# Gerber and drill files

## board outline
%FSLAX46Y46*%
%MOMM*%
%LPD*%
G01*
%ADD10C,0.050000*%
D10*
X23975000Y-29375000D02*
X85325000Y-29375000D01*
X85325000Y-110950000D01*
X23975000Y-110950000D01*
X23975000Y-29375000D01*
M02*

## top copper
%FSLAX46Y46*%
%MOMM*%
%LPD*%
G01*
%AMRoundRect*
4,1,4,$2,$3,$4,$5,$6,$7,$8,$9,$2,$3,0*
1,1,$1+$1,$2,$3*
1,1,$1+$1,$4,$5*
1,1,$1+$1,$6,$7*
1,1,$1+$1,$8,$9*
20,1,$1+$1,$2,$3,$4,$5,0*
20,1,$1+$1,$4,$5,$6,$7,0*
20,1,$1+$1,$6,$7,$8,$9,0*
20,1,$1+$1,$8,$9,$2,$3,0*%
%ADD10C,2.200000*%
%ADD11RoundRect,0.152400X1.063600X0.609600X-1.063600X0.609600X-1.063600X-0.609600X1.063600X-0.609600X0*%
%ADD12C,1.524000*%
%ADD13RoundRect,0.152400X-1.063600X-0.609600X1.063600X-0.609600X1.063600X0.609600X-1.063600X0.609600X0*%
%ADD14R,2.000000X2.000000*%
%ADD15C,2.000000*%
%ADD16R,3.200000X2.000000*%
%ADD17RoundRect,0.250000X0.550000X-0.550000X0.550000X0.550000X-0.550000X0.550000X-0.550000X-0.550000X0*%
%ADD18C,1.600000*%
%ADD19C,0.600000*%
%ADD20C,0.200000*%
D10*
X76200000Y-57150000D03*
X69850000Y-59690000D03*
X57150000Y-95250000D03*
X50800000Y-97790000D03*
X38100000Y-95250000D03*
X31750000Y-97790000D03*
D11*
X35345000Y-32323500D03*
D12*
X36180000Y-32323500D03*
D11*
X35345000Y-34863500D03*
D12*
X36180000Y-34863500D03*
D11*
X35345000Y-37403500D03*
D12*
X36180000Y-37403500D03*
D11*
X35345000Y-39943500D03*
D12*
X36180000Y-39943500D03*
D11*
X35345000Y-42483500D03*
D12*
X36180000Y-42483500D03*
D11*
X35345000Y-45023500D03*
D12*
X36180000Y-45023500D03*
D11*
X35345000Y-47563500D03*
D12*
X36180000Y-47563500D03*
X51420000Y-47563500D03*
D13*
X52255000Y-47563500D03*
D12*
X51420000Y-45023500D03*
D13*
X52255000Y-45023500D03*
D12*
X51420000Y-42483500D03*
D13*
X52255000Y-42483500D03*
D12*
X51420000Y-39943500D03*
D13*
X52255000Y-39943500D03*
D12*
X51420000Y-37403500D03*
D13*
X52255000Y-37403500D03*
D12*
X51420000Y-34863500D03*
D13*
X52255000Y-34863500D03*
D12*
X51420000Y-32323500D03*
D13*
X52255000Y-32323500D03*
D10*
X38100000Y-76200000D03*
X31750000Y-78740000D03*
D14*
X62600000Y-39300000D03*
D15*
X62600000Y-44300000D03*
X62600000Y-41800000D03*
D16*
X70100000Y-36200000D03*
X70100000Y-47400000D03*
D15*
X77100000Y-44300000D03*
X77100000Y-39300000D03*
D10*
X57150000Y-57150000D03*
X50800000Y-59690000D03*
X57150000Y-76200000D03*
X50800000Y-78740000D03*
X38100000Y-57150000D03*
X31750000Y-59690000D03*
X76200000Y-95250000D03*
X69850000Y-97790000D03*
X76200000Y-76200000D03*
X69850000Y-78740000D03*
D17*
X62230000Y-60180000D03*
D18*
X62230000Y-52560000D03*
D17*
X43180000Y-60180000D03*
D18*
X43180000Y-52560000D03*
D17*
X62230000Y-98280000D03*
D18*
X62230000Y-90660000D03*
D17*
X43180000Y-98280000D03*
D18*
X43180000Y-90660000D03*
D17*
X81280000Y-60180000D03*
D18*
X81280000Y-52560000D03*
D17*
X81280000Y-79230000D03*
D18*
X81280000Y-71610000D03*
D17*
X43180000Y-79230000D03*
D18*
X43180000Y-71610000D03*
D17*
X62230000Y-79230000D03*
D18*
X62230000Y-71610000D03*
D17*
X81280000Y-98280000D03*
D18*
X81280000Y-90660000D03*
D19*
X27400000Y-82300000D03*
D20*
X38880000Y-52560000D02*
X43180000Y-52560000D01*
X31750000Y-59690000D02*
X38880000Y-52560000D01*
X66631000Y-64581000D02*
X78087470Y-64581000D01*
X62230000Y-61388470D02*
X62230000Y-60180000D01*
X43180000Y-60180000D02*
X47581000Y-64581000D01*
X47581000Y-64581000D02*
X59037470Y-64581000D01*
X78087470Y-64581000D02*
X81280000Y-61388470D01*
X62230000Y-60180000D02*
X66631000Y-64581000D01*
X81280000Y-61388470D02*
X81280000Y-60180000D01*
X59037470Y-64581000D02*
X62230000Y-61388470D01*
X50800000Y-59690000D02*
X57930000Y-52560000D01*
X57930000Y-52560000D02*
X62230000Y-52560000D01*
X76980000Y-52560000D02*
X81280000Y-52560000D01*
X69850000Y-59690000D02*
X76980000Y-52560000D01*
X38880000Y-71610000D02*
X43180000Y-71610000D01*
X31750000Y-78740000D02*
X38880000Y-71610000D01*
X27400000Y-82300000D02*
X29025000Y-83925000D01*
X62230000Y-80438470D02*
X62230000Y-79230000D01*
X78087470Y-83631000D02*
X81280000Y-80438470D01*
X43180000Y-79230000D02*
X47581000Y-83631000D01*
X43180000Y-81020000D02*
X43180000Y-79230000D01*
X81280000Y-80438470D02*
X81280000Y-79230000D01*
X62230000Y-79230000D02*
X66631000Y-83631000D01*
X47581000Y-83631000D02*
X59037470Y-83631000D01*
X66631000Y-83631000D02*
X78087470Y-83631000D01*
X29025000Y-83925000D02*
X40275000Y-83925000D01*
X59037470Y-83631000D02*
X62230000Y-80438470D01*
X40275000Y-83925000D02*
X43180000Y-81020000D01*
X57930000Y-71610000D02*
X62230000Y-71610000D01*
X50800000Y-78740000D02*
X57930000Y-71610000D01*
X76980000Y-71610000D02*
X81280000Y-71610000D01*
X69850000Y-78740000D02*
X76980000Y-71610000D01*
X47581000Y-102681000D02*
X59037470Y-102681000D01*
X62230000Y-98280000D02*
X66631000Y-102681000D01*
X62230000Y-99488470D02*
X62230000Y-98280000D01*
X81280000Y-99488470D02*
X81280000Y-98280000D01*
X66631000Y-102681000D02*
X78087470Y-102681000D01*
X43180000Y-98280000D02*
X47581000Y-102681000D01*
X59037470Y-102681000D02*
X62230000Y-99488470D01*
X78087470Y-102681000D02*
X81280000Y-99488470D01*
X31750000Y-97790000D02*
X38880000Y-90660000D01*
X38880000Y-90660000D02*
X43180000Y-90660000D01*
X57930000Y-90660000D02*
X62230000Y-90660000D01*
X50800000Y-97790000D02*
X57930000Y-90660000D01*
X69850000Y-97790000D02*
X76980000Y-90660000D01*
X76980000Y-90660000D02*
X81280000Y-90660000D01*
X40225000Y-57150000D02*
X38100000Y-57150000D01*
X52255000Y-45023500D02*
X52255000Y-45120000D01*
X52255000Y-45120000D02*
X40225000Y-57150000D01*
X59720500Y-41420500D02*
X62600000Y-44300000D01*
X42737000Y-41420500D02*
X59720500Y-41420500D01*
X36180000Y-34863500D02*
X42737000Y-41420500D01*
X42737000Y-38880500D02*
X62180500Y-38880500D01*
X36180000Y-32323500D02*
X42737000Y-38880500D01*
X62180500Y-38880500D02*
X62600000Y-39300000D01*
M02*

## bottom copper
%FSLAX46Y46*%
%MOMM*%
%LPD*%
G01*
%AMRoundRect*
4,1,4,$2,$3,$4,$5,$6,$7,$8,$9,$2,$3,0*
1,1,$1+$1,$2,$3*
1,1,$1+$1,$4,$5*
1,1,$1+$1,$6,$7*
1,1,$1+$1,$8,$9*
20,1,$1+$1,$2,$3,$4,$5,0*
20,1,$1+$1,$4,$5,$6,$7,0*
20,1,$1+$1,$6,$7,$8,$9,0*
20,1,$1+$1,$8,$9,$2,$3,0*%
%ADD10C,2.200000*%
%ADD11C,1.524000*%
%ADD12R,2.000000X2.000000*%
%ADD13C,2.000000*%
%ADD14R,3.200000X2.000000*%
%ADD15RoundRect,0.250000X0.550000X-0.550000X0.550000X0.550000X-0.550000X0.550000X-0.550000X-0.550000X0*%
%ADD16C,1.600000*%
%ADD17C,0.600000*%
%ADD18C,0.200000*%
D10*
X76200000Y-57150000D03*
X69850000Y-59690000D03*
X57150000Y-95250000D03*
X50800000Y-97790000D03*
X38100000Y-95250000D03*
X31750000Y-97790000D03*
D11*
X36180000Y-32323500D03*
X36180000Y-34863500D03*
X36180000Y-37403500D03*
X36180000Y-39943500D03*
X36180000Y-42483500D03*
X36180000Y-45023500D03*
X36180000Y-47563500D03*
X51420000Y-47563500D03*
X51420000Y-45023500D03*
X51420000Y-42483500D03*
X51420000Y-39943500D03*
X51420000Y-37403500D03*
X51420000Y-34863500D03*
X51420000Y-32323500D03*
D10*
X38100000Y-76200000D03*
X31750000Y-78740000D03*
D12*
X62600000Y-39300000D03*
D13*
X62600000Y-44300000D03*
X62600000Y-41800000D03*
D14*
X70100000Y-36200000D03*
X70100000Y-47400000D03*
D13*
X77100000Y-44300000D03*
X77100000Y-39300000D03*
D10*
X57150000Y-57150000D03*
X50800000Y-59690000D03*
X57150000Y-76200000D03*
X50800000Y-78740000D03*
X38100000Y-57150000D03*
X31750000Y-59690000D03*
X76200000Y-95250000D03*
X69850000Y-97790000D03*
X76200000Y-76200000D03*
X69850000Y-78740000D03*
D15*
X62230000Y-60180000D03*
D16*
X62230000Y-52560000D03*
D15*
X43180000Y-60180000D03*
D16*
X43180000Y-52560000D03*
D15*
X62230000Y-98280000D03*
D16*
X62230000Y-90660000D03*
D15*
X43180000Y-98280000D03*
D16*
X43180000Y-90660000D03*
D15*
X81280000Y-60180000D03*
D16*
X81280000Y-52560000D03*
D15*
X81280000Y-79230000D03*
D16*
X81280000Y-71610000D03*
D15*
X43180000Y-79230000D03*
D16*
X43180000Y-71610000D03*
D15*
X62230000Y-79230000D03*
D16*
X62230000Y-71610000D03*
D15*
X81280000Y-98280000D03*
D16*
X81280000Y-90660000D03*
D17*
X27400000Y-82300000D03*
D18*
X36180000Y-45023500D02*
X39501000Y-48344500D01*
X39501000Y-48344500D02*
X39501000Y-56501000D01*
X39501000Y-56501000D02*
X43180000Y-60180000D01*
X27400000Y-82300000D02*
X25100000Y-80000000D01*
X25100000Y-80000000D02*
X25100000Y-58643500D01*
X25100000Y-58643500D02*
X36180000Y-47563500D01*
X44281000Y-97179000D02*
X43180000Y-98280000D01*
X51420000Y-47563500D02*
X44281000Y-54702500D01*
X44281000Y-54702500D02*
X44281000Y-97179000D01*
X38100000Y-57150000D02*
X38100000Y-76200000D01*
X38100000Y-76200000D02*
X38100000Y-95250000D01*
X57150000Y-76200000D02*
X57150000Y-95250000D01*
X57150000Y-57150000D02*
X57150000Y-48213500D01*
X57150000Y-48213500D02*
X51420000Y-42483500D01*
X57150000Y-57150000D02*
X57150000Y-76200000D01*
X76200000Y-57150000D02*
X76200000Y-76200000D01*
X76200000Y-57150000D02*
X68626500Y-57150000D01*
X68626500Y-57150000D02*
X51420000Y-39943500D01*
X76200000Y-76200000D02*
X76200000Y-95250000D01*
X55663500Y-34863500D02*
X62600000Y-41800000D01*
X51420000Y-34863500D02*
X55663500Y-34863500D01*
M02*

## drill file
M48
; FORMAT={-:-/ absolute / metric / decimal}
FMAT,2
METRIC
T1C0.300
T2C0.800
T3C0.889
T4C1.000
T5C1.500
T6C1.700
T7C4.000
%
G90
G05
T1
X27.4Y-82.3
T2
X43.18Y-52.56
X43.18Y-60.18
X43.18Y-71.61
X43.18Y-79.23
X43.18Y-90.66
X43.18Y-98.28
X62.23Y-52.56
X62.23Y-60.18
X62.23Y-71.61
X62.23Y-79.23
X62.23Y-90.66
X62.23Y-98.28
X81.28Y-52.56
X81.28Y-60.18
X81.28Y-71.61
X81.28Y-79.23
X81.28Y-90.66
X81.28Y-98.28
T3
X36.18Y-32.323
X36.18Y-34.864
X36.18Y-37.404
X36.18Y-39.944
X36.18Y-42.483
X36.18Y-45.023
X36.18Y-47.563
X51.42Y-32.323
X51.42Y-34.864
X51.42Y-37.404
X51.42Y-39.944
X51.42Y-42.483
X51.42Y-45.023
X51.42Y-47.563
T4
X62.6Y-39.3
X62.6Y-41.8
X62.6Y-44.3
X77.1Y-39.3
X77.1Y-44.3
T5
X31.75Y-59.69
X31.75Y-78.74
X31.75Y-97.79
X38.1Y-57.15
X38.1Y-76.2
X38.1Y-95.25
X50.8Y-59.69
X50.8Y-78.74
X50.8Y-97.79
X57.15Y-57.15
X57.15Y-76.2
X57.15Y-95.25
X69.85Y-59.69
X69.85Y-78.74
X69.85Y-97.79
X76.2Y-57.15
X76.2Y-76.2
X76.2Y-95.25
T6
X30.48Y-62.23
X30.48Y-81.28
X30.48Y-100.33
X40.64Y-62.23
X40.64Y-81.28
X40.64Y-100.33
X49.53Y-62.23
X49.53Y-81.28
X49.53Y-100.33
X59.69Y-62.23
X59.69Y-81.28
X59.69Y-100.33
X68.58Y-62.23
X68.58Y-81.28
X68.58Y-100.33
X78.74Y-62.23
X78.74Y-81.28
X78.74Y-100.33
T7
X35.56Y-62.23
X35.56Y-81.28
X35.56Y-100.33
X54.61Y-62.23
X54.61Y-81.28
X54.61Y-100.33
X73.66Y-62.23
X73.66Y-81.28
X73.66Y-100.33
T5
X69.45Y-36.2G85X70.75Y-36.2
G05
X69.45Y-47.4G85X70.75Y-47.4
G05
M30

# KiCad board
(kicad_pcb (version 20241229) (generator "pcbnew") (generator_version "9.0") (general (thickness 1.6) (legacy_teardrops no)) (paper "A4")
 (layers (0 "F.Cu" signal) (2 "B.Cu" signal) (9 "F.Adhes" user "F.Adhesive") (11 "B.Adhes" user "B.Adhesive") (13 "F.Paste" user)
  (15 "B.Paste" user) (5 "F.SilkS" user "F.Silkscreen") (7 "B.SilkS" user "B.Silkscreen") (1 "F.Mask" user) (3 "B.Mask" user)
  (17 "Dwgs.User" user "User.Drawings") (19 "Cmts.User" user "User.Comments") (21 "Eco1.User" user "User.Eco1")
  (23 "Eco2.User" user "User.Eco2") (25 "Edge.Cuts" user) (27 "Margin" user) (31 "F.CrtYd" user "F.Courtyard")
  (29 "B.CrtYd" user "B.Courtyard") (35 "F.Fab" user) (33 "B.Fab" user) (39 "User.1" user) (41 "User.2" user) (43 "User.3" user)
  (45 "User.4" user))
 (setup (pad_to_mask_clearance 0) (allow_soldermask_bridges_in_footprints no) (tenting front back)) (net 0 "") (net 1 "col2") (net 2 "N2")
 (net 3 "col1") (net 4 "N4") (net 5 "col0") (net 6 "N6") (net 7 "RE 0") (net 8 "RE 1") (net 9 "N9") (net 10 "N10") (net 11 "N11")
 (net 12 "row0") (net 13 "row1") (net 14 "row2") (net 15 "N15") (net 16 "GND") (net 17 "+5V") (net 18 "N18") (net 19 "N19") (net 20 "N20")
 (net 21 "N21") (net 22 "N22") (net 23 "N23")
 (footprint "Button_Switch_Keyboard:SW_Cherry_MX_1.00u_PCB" (layer "F.Cu") (at 76.2 57.15)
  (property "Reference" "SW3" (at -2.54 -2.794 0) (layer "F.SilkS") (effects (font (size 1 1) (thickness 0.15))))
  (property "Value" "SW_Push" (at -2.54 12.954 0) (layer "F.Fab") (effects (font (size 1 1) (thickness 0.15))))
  (pad "" np_thru_hole circle (at -7.62 5.08) (size 1.7 1.7) (drill 1.7) (layers "*.Cu" "*.Mask"))
  (pad "" np_thru_hole circle (at -2.54 5.08) (size 4 4) (drill 4) (layers "*.Cu" "*.Mask"))
  (pad "" np_thru_hole circle (at 2.54 5.08) (size 1.7 1.7) (drill 1.7) (layers "*.Cu" "*.Mask"))
  (pad "1" thru_hole circle (at 0 0) (size 2.2 2.2) (drill 1.5) (layers "*.Cu" "*.Mask") (remove_unused_layers no) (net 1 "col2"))
  (pad "2" thru_hole circle (at -6.35 2.54) (size 2.2 2.2) (drill 1.5) (layers "*.Cu" "*.Mask") (remove_unused_layers no) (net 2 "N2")))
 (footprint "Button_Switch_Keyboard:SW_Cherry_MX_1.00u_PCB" (layer "F.Cu") (at 57.15 95.25)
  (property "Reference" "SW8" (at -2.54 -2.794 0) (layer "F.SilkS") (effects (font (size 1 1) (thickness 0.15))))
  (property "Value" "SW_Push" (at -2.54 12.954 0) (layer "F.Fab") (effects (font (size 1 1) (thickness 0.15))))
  (pad "" np_thru_hole circle (at -7.62 5.08) (size 1.7 1.7) (drill 1.7) (layers "*.Cu" "*.Mask"))
  (pad "" np_thru_hole circle (at -2.54 5.08) (size 4 4) (drill 4) (layers "*.Cu" "*.Mask"))
  (pad "" np_thru_hole circle (at 2.54 5.08) (size 1.7 1.7) (drill 1.7) (layers "*.Cu" "*.Mask"))
  (pad "1" thru_hole circle (at 0 0) (size 2.2 2.2) (drill 1.5) (layers "*.Cu" "*.Mask") (remove_unused_layers no) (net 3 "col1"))
  (pad "2" thru_hole circle (at -6.35 2.54) (size 2.2 2.2) (drill 1.5) (layers "*.Cu" "*.Mask") (remove_unused_layers no) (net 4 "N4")))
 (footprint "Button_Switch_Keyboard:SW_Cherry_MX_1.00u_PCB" (layer "F.Cu") (at 38.1 95.25)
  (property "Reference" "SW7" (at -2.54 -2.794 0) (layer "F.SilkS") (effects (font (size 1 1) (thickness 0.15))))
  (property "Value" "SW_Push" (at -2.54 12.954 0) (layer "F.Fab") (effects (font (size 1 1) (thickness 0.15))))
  (pad "" np_thru_hole circle (at -7.62 5.08) (size 1.7 1.7) (drill 1.7) (layers "*.Cu" "*.Mask"))
  (pad "" np_thru_hole circle (at -2.54 5.08) (size 4 4) (drill 4) (layers "*.Cu" "*.Mask"))
  (pad "" np_thru_hole circle (at 2.54 5.08) (size 1.7 1.7) (drill 1.7) (layers "*.Cu" "*.Mask"))
  (pad "1" thru_hole circle (at 0 0) (size 2.2 2.2) (drill 1.5) (layers "*.Cu" "*.Mask") (remove_unused_layers no) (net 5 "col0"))
  (pad "2" thru_hole circle (at -6.35 2.54) (size 2.2 2.2) (drill 1.5) (layers "*.Cu" "*.Mask") (remove_unused_layers no) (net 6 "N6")))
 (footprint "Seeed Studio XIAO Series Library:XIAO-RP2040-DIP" (layer "F.Cu") (at 43.8 39.9435)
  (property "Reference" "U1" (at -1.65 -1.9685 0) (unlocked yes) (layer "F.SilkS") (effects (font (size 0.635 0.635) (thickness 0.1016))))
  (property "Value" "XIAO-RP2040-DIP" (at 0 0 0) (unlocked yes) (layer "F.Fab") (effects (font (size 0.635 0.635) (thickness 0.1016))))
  (pad "1" smd roundrect (at -8.455 -7.62 180) (size 2.432 1.524) (layers "F.Cu" "F.Mask") (roundrect_rratio 0.1) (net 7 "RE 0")
   (thermal_bridge_angle 45))
  (pad "1" thru_hole circle (at -7.62 -7.62 180) (size 1.524 1.524) (drill 0.889) (layers "*.Cu" "*.Mask") (remove_unused_layers no)
   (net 7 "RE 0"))
  (pad "2" smd roundrect (at -8.455 -5.08 180) (size 2.432 1.524) (layers "F.Cu" "F.Mask") (roundrect_rratio 0.1) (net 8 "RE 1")
   (thermal_bridge_angle 45))
  (pad "2" thru_hole circle (at -7.62 -5.08 180) (size 1.524 1.524) (drill 0.889) (layers "*.Cu" "*.Mask") (remove_unused_layers no)
   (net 8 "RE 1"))
  (pad "3" smd roundrect (at -8.455 -2.54 180) (size 2.432 1.524) (layers "F.Cu" "F.Mask") (roundrect_rratio 0.1) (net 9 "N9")
   (thermal_bridge_angle 45))
  (pad "3" thru_hole circle (at -7.62 -2.54 180) (size 1.524 1.524) (drill 0.889) (layers "*.Cu" "*.Mask") (remove_unused_layers no)
   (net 9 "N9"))
  (pad "4" smd roundrect (at -8.455 0 180) (size 2.432 1.524) (layers "F.Cu" "F.Mask") (roundrect_rratio 0.1) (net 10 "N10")
   (thermal_bridge_angle 45))
  (pad "4" thru_hole circle (at -7.62 0 180) (size 1.524 1.524) (drill 0.889) (layers "*.Cu" "*.Mask") (remove_unused_layers no)
   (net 10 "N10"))
  (pad "5" smd roundrect (at -8.455 2.54 180) (size 2.432 1.524) (layers "F.Cu" "F.Mask") (roundrect_rratio 0.1) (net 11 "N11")
   (thermal_bridge_angle 45))
  (pad "5" thru_hole circle (at -7.62 2.54 180) (size 1.524 1.524) (drill 0.889) (layers "*.Cu" "*.Mask") (remove_unused_layers no)
   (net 11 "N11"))
  (pad "6" smd roundrect (at -8.455 5.08 180) (size 2.432 1.524) (layers "F.Cu" "F.Mask") (roundrect_rratio 0.1) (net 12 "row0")
   (thermal_bridge_angle 45))
  (pad "6" thru_hole circle (at -7.62 5.08 180) (size 1.524 1.524) (drill 0.889) (layers "*.Cu" "*.Mask") (remove_unused_layers no)
   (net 12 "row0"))
  (pad "7" smd roundrect (at -8.455 7.62 180) (size 2.432 1.524) (layers "F.Cu" "F.Mask") (roundrect_rratio 0.1) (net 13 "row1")
   (thermal_bridge_angle 45))
  (pad "7" thru_hole circle (at -7.62 7.62 180) (size 1.524 1.524) (drill 0.889) (layers "*.Cu" "*.Mask") (remove_unused_layers no)
   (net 13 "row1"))
  (pad "8" thru_hole circle (at 7.62 7.62) (size 1.524 1.524) (drill 0.889) (layers "*.Cu" "*.Mask") (remove_unused_layers no)
   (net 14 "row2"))
  (pad "8" smd roundrect (at 8.455 7.62) (size 2.432 1.524) (layers "F.Cu" "F.Mask") (roundrect_rratio 0.1) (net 14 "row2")
   (thermal_bridge_angle 45))
  (pad "9" thru_hole circle (at 7.62 5.08) (size 1.524 1.524) (drill 0.889) (layers "*.Cu" "*.Mask") (remove_unused_layers no)
   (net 5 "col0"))
  (pad "9" smd roundrect (at 8.455 5.08) (size 2.432 1.524) (layers "F.Cu" "F.Mask") (roundrect_rratio 0.1) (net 5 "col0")
   (thermal_bridge_angle 45))
  (pad "10" thru_hole circle (at 7.62 2.54) (size 1.524 1.524) (drill 0.889) (layers "*.Cu" "*.Mask") (remove_unused_layers no)
   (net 3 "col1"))
  (pad "10" smd roundrect (at 8.455 2.54) (size 2.432 1.524) (layers "F.Cu" "F.Mask") (roundrect_rratio 0.1) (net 3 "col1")
   (thermal_bridge_angle 45))
  (pad "11" thru_hole circle (at 7.62 0) (size 1.524 1.524) (drill 0.889) (layers "*.Cu" "*.Mask") (remove_unused_layers no) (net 1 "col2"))
  (pad "11" smd roundrect (at 8.455 0) (size 2.432 1.524) (layers "F.Cu" "F.Mask") (roundrect_rratio 0.1) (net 1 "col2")
   (thermal_bridge_angle 45))
  (pad "12" thru_hole circle (at 7.62 -2.54) (size 1.524 1.524) (drill 0.889) (layers "*.Cu" "*.Mask") (remove_unused_layers no)
   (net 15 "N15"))
  (pad "12" smd roundrect (at 8.455 -2.54) (size 2.432 1.524) (layers "F.Cu" "F.Mask") (roundrect_rratio 0.1) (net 15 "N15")
   (thermal_bridge_angle 45))
  (pad "13" thru_hole circle (at 7.62 -5.08) (size 1.524 1.524) (drill 0.889) (layers "*.Cu" "*.Mask") (remove_unused_layers no)
   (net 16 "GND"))
  (pad "13" smd roundrect (at 8.455 -5.08) (size 2.432 1.524) (layers "F.Cu" "F.Mask") (roundrect_rratio 0.1) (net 16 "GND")
   (thermal_bridge_angle 45))
  (pad "14" thru_hole circle (at 7.62 -7.62) (size 1.524 1.524) (drill 0.889) (layers "*.Cu" "*.Mask") (remove_unused_layers no)
   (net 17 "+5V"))
  (pad "14" smd roundrect (at 8.455 -7.62) (size 2.432 1.524) (layers "F.Cu" "F.Mask") (roundrect_rratio 0.1) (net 17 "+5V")
   (thermal_bridge_angle 45)))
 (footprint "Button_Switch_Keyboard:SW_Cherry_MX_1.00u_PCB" (layer "F.Cu") (at 38.1 76.2)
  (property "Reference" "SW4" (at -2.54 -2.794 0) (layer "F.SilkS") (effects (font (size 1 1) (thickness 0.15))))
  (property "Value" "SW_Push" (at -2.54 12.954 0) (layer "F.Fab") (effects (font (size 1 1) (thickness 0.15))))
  (pad "" np_thru_hole circle (at -7.62 5.08) (size 1.7 1.7) (drill 1.7) (layers "*.Cu" "*.Mask"))
  (pad "" np_thru_hole circle (at -2.54 5.08) (size 4 4) (drill 4) (layers "*.Cu" "*.Mask"))
  (pad "" np_thru_hole circle (at 2.54 5.08) (size 1.7 1.7) (drill 1.7) (layers "*.Cu" "*.Mask"))
  (pad "1" thru_hole circle (at 0 0) (size 2.2 2.2) (drill 1.5) (layers "*.Cu" "*.Mask") (remove_unused_layers no) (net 5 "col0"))
  (pad "2" thru_hole circle (at -6.35 2.54) (size 2.2 2.2) (drill 1.5) (layers "*.Cu" "*.Mask") (remove_unused_layers no) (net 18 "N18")))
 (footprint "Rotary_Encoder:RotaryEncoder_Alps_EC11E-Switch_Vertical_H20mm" (layer "F.Cu") (at 62.6 39.3)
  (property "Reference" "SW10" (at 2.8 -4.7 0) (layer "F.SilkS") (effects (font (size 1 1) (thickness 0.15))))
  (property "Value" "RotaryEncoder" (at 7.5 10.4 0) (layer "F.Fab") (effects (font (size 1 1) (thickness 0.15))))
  (pad "A" thru_hole rect (at 0 0) (size 2 2) (drill 1) (layers "*.Cu" "*.Mask") (remove_unused_layers no) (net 7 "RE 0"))
  (pad "B" thru_hole circle (at 0 5) (size 2 2) (drill 1) (layers "*.Cu" "*.Mask") (remove_unused_layers no) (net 8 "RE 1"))
  (pad "C" thru_hole circle (at 0 2.5) (size 2 2) (drill 1) (layers "*.Cu" "*.Mask") (remove_unused_layers no) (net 16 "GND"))
  (pad "MP" thru_hole rect (at 7.5 -3.1) (size 3.2 2) (drill oval 2.8 1.5) (layers "*.Cu" "*.Mask") (remove_unused_layers no))
  (pad "MP" thru_hole rect (at 7.5 8.1) (size 3.2 2) (drill oval 2.8 1.5) (layers "*.Cu" "*.Mask") (remove_unused_layers no))
  (pad "S1" thru_hole circle (at 14.5 5) (size 2 2) (drill 1) (layers "*.Cu" "*.Mask") (remove_unused_layers no))
  (pad "S2" thru_hole circle (at 14.5 0) (size 2 2) (drill 1) (layers "*.Cu" "*.Mask") (remove_unused_layers no)))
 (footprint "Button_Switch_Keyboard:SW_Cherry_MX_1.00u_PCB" (layer "F.Cu") (at 57.15 57.15)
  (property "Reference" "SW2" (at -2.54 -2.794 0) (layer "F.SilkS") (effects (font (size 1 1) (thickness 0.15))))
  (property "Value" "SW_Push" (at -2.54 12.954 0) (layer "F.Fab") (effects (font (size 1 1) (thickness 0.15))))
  (pad "" np_thru_hole circle (at -7.62 5.08) (size 1.7 1.7) (drill 1.7) (layers "*.Cu" "*.Mask"))
  (pad "" np_thru_hole circle (at -2.54 5.08) (size 4 4) (drill 4) (layers "*.Cu" "*.Mask"))
  (pad "" np_thru_hole circle (at 2.54 5.08) (size 1.7 1.7) (drill 1.7) (layers "*.Cu" "*.Mask"))
  (pad "1" thru_hole circle (at 0 0) (size 2.2 2.2) (drill 1.5) (layers "*.Cu" "*.Mask") (remove_unused_layers no) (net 3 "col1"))
  (pad "2" thru_hole circle (at -6.35 2.54) (size 2.2 2.2) (drill 1.5) (layers "*.Cu" "*.Mask") (remove_unused_layers no) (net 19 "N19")))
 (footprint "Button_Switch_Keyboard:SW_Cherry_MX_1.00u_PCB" (layer "F.Cu") (at 57.15 76.2)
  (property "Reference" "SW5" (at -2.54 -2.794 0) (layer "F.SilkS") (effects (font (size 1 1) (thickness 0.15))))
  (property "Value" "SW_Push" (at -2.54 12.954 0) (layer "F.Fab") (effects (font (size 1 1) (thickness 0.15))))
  (pad "" np_thru_hole circle (at -7.62 5.08) (size 1.7 1.7) (drill 1.7) (layers "*.Cu" "*.Mask"))
  (pad "" np_thru_hole circle (at -2.54 5.08) (size 4 4) (drill 4) (layers "*.Cu" "*.Mask"))
  (pad "" np_thru_hole circle (at 2.54 5.08) (size 1.7 1.7) (drill 1.7) (layers "*.Cu" "*.Mask"))
  (pad "1" thru_hole circle (at 0 0) (size 2.2 2.2) (drill 1.5) (layers "*.Cu" "*.Mask") (remove_unused_layers no) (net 3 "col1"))
  (pad "2" thru_hole circle (at -6.35 2.54) (size 2.2 2.2) (drill 1.5) (layers "*.Cu" "*.Mask") (remove_unused_layers no) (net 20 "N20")))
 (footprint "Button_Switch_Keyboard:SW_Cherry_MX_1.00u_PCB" (layer "F.Cu") (at 38.1 57.15)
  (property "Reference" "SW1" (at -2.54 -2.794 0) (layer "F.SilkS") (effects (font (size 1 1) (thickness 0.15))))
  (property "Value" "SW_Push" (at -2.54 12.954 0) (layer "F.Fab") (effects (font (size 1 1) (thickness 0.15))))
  (pad "" np_thru_hole circle (at -7.62 5.08) (size 1.7 1.7) (drill 1.7) (layers "*.Cu" "*.Mask"))
  (pad "" np_thru_hole circle (at -2.54 5.08) (size 4 4) (drill 4) (layers "*.Cu" "*.Mask"))
  (pad "" np_thru_hole circle (at 2.54 5.08) (size 1.7 1.7) (drill 1.7) (layers "*.Cu" "*.Mask"))
  (pad "1" thru_hole circle (at 0 0) (size 2.2 2.2) (drill 1.5) (layers "*.Cu" "*.Mask") (remove_unused_layers no) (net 5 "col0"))
  (pad "2" thru_hole circle (at -6.35 2.54) (size 2.2 2.2) (drill 1.5) (layers "*.Cu" "*.Mask") (remove_unused_layers no) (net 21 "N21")))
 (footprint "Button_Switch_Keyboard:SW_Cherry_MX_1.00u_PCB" (layer "F.Cu") (at 76.2 95.25)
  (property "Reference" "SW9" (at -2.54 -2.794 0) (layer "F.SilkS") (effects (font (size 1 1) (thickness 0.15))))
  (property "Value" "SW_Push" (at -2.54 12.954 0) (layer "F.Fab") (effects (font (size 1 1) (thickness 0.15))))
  (pad "" np_thru_hole circle (at -7.62 5.08) (size 1.7 1.7) (drill 1.7) (layers "*.Cu" "*.Mask"))
  (pad "" np_thru_hole circle (at -2.54 5.08) (size 4 4) (drill 4) (layers "*.Cu" "*.Mask"))
  (pad "" np_thru_hole circle (at 2.54 5.08) (size 1.7 1.7) (drill 1.7) (layers "*.Cu" "*.Mask"))
  (pad "1" thru_hole circle (at 0 0) (size 2.2 2.2) (drill 1.5) (layers "*.Cu" "*.Mask") (remove_unused_layers no) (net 1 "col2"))
  (pad "2" thru_hole circle (at -6.35 2.54) (size 2.2 2.2) (drill 1.5) (layers "*.Cu" "*.Mask") (remove_unused_layers no) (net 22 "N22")))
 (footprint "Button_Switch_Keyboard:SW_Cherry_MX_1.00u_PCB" (layer "F.Cu") (at 76.2 76.2)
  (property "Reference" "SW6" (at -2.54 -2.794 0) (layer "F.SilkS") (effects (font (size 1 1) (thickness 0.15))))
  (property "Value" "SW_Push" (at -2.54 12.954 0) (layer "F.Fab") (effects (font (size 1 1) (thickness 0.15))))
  (pad "" np_thru_hole circle (at -7.62 5.08) (size 1.7 1.7) (drill 1.7) (layers "*.Cu" "*.Mask"))
  (pad "" np_thru_hole circle (at -2.54 5.08) (size 4 4) (drill 4) (layers "*.Cu" "*.Mask"))
  (pad "" np_thru_hole circle (at 2.54 5.08) (size 1.7 1.7) (drill 1.7) (layers "*.Cu" "*.Mask"))
  (pad "1" thru_hole circle (at 0 0) (size 2.2 2.2) (drill 1.5) (layers "*.Cu" "*.Mask") (remove_unused_layers no) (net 1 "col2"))
  (pad "2" thru_hole circle (at -6.35 2.54) (size 2.2 2.2) (drill 1.5) (layers "*.Cu" "*.Mask") (remove_unused_layers no) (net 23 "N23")))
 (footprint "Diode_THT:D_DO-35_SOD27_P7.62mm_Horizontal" (layer "B.Cu") (at 62.23 60.18 90)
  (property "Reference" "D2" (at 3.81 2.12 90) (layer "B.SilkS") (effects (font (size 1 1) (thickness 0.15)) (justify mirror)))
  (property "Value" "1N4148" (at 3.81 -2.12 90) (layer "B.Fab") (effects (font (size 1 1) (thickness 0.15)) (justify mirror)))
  (pad "1" thru_hole roundrect (at 0 0 90) (size 1.6 1.6) (drill 0.8) (layers "*.Cu" "*.Mask") (remove_unused_layers no)
   (roundrect_rratio 0.15625) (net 12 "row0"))
  (pad "2" thru_hole circle (at 7.62 0 90) (size 1.6 1.6) (drill 0.8) (layers "*.Cu" "*.Mask") (remove_unused_layers no) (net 19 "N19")))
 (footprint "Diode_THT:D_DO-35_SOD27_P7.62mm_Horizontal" (layer "B.Cu") (at 43.18 60.18 90)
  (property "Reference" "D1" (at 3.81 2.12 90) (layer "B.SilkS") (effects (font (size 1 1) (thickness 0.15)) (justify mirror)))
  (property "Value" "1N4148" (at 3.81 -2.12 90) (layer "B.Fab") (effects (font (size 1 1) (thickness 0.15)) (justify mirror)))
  (pad "1" thru_hole roundrect (at 0 0 90) (size 1.6 1.6) (drill 0.8) (layers "*.Cu" "*.Mask") (remove_unused_layers no)
   (roundrect_rratio 0.15625) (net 12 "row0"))
  (pad "2" thru_hole circle (at 7.62 0 90) (size 1.6 1.6) (drill 0.8) (layers "*.Cu" "*.Mask") (remove_unused_layers no) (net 21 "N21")))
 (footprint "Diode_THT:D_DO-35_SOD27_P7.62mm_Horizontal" (layer "B.Cu") (at 62.23 98.28 90)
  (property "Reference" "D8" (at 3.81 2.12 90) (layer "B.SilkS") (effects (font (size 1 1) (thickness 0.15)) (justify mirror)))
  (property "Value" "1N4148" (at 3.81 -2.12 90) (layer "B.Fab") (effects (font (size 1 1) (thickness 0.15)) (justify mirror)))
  (pad "1" thru_hole roundrect (at 0 0 90) (size 1.6 1.6) (drill 0.8) (layers "*.Cu" "*.Mask") (remove_unused_layers no)
   (roundrect_rratio 0.15625) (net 14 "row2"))
  (pad "2" thru_hole circle (at 7.62 0 90) (size 1.6 1.6) (drill 0.8) (layers "*.Cu" "*.Mask") (remove_unused_layers no) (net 4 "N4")))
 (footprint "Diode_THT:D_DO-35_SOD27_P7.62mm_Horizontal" (layer "B.Cu") (at 43.18 98.28 90)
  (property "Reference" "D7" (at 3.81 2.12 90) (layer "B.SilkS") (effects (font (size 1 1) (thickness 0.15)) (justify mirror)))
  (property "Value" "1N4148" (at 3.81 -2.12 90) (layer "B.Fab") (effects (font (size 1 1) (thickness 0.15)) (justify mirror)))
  (pad "1" thru_hole roundrect (at 0 0 90) (size 1.6 1.6) (drill 0.8) (layers "*.Cu" "*.Mask") (remove_unused_layers no)
   (roundrect_rratio 0.15625) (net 14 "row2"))
  (pad "2" thru_hole circle (at 7.62 0 90) (size 1.6 1.6) (drill 0.8) (layers "*.Cu" "*.Mask") (remove_unused_layers no) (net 6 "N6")))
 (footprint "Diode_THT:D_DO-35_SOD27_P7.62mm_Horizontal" (layer "B.Cu") (at 81.28 60.18 90)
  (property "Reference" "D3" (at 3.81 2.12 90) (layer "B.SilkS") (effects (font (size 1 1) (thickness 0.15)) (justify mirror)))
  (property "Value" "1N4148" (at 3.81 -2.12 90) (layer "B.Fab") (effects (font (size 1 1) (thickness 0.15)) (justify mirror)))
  (pad "1" thru_hole roundrect (at 0 0 90) (size 1.6 1.6) (drill 0.8) (layers "*.Cu" "*.Mask") (remove_unused_layers no)
   (roundrect_rratio 0.15625) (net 12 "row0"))
  (pad "2" thru_hole circle (at 7.62 0 90) (size 1.6 1.6) (drill 0.8) (layers "*.Cu" "*.Mask") (remove_unused_layers no) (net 2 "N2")))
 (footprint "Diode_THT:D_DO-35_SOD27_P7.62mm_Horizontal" (layer "B.Cu") (at 81.28 79.23 90)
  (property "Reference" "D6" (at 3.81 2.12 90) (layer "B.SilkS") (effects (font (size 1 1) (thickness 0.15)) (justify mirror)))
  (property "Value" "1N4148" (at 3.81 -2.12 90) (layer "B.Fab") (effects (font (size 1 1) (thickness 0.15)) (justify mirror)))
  (pad "1" thru_hole roundrect (at 0 0 90) (size 1.6 1.6) (drill 0.8) (layers "*.Cu" "*.Mask") (remove_unused_layers no)
   (roundrect_rratio 0.15625) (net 13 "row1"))
  (pad "2" thru_hole circle (at 7.62 0 90) (size 1.6 1.6) (drill 0.8) (layers "*.Cu" "*.Mask") (remove_unused_layers no) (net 23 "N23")))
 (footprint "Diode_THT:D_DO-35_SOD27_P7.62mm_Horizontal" (layer "B.Cu") (at 43.18 79.23 90)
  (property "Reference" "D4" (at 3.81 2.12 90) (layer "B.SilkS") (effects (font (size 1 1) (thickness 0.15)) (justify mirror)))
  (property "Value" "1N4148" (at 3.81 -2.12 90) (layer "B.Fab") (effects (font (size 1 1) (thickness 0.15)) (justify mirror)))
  (pad "1" thru_hole roundrect (at 0 0 90) (size 1.6 1.6) (drill 0.8) (layers "*.Cu" "*.Mask") (remove_unused_layers no)
   (roundrect_rratio 0.15625) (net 13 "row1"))
  (pad "2" thru_hole circle (at 7.62 0 90) (size 1.6 1.6) (drill 0.8) (layers "*.Cu" "*.Mask") (remove_unused_layers no) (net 18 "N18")))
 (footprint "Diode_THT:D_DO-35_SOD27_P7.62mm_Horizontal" (layer "B.Cu") (at 62.23 79.23 90)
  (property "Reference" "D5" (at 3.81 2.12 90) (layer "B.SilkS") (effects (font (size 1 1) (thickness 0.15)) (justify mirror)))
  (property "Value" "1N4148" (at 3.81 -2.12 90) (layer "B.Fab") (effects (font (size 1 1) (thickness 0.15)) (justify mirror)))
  (pad "1" thru_hole roundrect (at 0 0 90) (size 1.6 1.6) (drill 0.8) (layers "*.Cu" "*.Mask") (remove_unused_layers no)
   (roundrect_rratio 0.15625) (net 13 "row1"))
  (pad "2" thru_hole circle (at 7.62 0 90) (size 1.6 1.6) (drill 0.8) (layers "*.Cu" "*.Mask") (remove_unused_layers no) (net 20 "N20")))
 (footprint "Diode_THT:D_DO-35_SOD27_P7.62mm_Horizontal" (layer "B.Cu") (at 81.28 98.28 90)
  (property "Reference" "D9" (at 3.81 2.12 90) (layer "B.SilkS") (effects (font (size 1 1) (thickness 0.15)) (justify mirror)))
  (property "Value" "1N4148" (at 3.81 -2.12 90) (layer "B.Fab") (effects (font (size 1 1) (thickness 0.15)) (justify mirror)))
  (pad "1" thru_hole roundrect (at 0 0 90) (size 1.6 1.6) (drill 0.8) (layers "*.Cu" "*.Mask") (remove_unused_layers no)
   (roundrect_rratio 0.15625) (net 14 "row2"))
  (pad "2" thru_hole circle (at 7.62 0 90) (size 1.6 1.6) (drill 0.8) (layers "*.Cu" "*.Mask") (remove_unused_layers no) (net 22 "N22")))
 (gr_rect (start 23.975 29.375) (end 85.325 110.95) (stroke (width 0.05) (type default)) (fill no) (layer "Edge.Cuts"))
 (segment (start 38.88 52.56) (end 43.18 52.56) (width 0.2) (layer "F.Cu") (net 21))
 (segment (start 31.75 59.69) (end 38.88 52.56) (width 0.2) (layer "F.Cu") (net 21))
 (segment (start 66.631 64.581) (end 78.08747 64.581) (width 0.2) (layer "F.Cu") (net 12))
 (segment (start 62.23 61.38847) (end 62.23 60.18) (width 0.2) (layer "F.Cu") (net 12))
 (segment (start 43.18 60.18) (end 47.581 64.581) (width 0.2) (layer "F.Cu") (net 12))
 (segment (start 47.581 64.581) (end 59.03747 64.581) (width 0.2) (layer "F.Cu") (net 12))
 (segment (start 78.08747 64.581) (end 81.28 61.38847) (width 0.2) (layer "F.Cu") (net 12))
 (segment (start 62.23 60.18) (end 66.631 64.581) (width 0.2) (layer "F.Cu") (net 12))
 (segment (start 81.28 61.38847) (end 81.28 60.18) (width 0.2) (layer "F.Cu") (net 12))
 (segment (start 59.03747 64.581) (end 62.23 61.38847) (width 0.2) (layer "F.Cu") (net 12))
 (segment (start 36.18 45.0235) (end 39.501 48.3445) (width 0.2) (layer "B.Cu") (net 12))
 (segment (start 39.501 48.3445) (end 39.501 56.501) (width 0.2) (layer "B.Cu") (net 12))
 (segment (start 39.501 56.501) (end 43.18 60.18) (width 0.2) (layer "B.Cu") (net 12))
 (segment (start 50.8 59.69) (end 57.93 52.56) (width 0.2) (layer "F.Cu") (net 19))
 (segment (start 57.93 52.56) (end 62.23 52.56) (width 0.2) (layer "F.Cu") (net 19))
 (segment (start 76.98 52.56) (end 81.28 52.56) (width 0.2) (layer "F.Cu") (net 2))
 (segment (start 69.85 59.69) (end 76.98 52.56) (width 0.2) (layer "F.Cu") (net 2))
 (segment (start 38.88 71.61) (end 43.18 71.61) (width 0.2) (layer "F.Cu") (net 18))
 (segment (start 31.75 78.74) (end 38.88 71.61) (width 0.2) (layer "F.Cu") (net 18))
 (segment (start 27.4 82.3) (end 29.025 83.925) (width 0.2) (layer "F.Cu") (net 13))
 (segment (start 62.23 80.43847) (end 62.23 79.23) (width 0.2) (layer "F.Cu") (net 13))
 (segment (start 78.08747 83.631) (end 81.28 80.43847) (width 0.2) (layer "F.Cu") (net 13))
 (segment (start 43.18 79.23) (end 47.581 83.631) (width 0.2) (layer "F.Cu") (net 13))
 (segment (start 43.18 81.02) (end 43.18 79.23) (width 0.2) (layer "F.Cu") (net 13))
 (segment (start 81.28 80.43847) (end 81.28 79.23) (width 0.2) (layer "F.Cu") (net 13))
 (segment (start 62.23 79.23) (end 66.631 83.631) (width 0.2) (layer "F.Cu") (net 13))
 (segment (start 47.581 83.631) (end 59.03747 83.631) (width 0.2) (layer "F.Cu") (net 13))
 (segment (start 66.631 83.631) (end 78.08747 83.631) (width 0.2) (layer "F.Cu") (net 13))
 (segment (start 29.025 83.925) (end 40.275 83.925) (width 0.2) (layer "F.Cu") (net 13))
 (segment (start 59.03747 83.631) (end 62.23 80.43847) (width 0.2) (layer "F.Cu") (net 13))
 (segment (start 40.275 83.925) (end 43.18 81.02) (width 0.2) (layer "F.Cu") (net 13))
 (via (at 27.4 82.3) (size 0.6) (drill 0.3) (layers "F.Cu" "B.Cu") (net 13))
 (segment (start 27.4 82.3) (end 25.1 80) (width 0.2) (layer "B.Cu") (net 13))
 (segment (start 25.1 80) (end 25.1 58.6435) (width 0.2) (layer "B.Cu") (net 13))
 (segment (start 25.1 58.6435) (end 36.18 47.5635) (width 0.2) (layer "B.Cu") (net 13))
 (segment (start 57.93 71.61) (end 62.23 71.61) (width 0.2) (layer "F.Cu") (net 20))
 (segment (start 50.8 78.74) (end 57.93 71.61) (width 0.2) (layer "F.Cu") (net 20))
 (segment (start 76.98 71.61) (end 81.28 71.61) (width 0.2) (layer "F.Cu") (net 23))
 (segment (start 69.85 78.74) (end 76.98 71.61) (width 0.2) (layer "F.Cu") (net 23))
 (segment (start 47.581 102.681) (end 59.03747 102.681) (width 0.2) (layer "F.Cu") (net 14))
 (segment (start 62.23 98.28) (end 66.631 102.681) (width 0.2) (layer "F.Cu") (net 14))
 (segment (start 62.23 99.48847) (end 62.23 98.28) (width 0.2) (layer "F.Cu") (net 14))
 (segment (start 81.28 99.48847) (end 81.28 98.28) (width 0.2) (layer "F.Cu") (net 14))
 (segment (start 66.631 102.681) (end 78.08747 102.681) (width 0.2) (layer "F.Cu") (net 14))
 (segment (start 43.18 98.28) (end 47.581 102.681) (width 0.2) (layer "F.Cu") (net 14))
 (segment (start 59.03747 102.681) (end 62.23 99.48847) (width 0.2) (layer "F.Cu") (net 14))
 (segment (start 78.08747 102.681) (end 81.28 99.48847) (width 0.2) (layer "F.Cu") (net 14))
 (segment (start 44.281 97.179) (end 43.18 98.28) (width 0.2) (layer "B.Cu") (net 14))
 (segment (start 51.42 47.5635) (end 44.281 54.7025) (width 0.2) (layer "B.Cu") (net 14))
 (segment (start 44.281 54.7025) (end 44.281 97.179) (width 0.2) (layer "B.Cu") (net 14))
 (segment (start 31.75 97.79) (end 38.88 90.66) (width 0.2) (layer "F.Cu") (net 6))
 (segment (start 38.88 90.66) (end 43.18 90.66) (width 0.2) (layer "F.Cu") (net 6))
 (segment (start 57.93 90.66) (end 62.23 90.66) (width 0.2) (layer "F.Cu") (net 4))
 (segment (start 50.8 97.79) (end 57.93 90.66) (width 0.2) (layer "F.Cu") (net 4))
 (segment (start 69.85 97.79) (end 76.98 90.66) (width 0.2) (layer "F.Cu") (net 22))
 (segment (start 76.98 90.66) (end 81.28 90.66) (width 0.2) (layer "F.Cu") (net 22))
 (segment (start 40.225 57.15) (end 38.1 57.15) (width 0.2) (layer "F.Cu") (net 5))
 (segment (start 52.255 45.0235) (end 52.255 45.12) (width 0.2) (layer "F.Cu") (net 5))
 (segment (start 52.255 45.12) (end 40.225 57.15) (width 0.2) (layer "F.Cu") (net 5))
 (segment (start 38.1 57.15) (end 38.1 76.2) (width 0.2) (layer "B.Cu") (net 5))
 (segment (start 38.1 76.2) (end 38.1 95.25) (width 0.2) (layer "B.Cu") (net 5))
 (segment (start 57.15 76.2) (end 57.15 95.25) (width 0.2) (layer "B.Cu") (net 3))
 (segment (start 57.15 57.15) (end 57.15 48.2135) (width 0.2) (layer "B.Cu") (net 3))
 (segment (start 57.15 48.2135) (end 51.42 42.4835) (width 0.2) (layer "B.Cu") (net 3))
 (segment (start 57.15 57.15) (end 57.15 76.2) (width 0.2) (layer "B.Cu") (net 3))
 (segment (start 76.2 57.15) (end 76.2 76.2) (width 0.2) (layer "B.Cu") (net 1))
 (segment (start 76.2 57.15) (end 68.6265 57.15) (width 0.2) (layer "B.Cu") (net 1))
 (segment (start 68.6265 57.15) (end 51.42 39.9435) (width 0.2) (layer "B.Cu") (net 1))
 (segment (start 76.2 76.2) (end 76.2 95.25) (width 0.2) (layer "B.Cu") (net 1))
 (segment (start 55.6635 34.8635) (end 62.6 41.8) (width 0.2) (layer "B.Cu") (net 16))
 (segment (start 51.42 34.8635) (end 55.6635 34.8635) (width 0.2) (layer "B.Cu") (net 16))
 (segment (start 59.7205 41.4205) (end 62.6 44.3) (width 0.2) (layer "F.Cu") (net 8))
 (segment (start 42.737 41.4205) (end 59.7205 41.4205) (width 0.2) (layer "F.Cu") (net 8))
 (segment (start 36.18 34.8635) (end 42.737 41.4205) (width 0.2) (layer "F.Cu") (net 8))
 (segment (start 42.737 38.8805) (end 62.1805 38.8805) (width 0.2) (layer "F.Cu") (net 7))
 (segment (start 36.18 32.3235) (end 42.737 38.8805) (width 0.2) (layer "F.Cu") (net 7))
 (segment (start 62.1805 38.8805) (end 62.6 39.3) (width 0.2) (layer "F.Cu") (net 7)))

